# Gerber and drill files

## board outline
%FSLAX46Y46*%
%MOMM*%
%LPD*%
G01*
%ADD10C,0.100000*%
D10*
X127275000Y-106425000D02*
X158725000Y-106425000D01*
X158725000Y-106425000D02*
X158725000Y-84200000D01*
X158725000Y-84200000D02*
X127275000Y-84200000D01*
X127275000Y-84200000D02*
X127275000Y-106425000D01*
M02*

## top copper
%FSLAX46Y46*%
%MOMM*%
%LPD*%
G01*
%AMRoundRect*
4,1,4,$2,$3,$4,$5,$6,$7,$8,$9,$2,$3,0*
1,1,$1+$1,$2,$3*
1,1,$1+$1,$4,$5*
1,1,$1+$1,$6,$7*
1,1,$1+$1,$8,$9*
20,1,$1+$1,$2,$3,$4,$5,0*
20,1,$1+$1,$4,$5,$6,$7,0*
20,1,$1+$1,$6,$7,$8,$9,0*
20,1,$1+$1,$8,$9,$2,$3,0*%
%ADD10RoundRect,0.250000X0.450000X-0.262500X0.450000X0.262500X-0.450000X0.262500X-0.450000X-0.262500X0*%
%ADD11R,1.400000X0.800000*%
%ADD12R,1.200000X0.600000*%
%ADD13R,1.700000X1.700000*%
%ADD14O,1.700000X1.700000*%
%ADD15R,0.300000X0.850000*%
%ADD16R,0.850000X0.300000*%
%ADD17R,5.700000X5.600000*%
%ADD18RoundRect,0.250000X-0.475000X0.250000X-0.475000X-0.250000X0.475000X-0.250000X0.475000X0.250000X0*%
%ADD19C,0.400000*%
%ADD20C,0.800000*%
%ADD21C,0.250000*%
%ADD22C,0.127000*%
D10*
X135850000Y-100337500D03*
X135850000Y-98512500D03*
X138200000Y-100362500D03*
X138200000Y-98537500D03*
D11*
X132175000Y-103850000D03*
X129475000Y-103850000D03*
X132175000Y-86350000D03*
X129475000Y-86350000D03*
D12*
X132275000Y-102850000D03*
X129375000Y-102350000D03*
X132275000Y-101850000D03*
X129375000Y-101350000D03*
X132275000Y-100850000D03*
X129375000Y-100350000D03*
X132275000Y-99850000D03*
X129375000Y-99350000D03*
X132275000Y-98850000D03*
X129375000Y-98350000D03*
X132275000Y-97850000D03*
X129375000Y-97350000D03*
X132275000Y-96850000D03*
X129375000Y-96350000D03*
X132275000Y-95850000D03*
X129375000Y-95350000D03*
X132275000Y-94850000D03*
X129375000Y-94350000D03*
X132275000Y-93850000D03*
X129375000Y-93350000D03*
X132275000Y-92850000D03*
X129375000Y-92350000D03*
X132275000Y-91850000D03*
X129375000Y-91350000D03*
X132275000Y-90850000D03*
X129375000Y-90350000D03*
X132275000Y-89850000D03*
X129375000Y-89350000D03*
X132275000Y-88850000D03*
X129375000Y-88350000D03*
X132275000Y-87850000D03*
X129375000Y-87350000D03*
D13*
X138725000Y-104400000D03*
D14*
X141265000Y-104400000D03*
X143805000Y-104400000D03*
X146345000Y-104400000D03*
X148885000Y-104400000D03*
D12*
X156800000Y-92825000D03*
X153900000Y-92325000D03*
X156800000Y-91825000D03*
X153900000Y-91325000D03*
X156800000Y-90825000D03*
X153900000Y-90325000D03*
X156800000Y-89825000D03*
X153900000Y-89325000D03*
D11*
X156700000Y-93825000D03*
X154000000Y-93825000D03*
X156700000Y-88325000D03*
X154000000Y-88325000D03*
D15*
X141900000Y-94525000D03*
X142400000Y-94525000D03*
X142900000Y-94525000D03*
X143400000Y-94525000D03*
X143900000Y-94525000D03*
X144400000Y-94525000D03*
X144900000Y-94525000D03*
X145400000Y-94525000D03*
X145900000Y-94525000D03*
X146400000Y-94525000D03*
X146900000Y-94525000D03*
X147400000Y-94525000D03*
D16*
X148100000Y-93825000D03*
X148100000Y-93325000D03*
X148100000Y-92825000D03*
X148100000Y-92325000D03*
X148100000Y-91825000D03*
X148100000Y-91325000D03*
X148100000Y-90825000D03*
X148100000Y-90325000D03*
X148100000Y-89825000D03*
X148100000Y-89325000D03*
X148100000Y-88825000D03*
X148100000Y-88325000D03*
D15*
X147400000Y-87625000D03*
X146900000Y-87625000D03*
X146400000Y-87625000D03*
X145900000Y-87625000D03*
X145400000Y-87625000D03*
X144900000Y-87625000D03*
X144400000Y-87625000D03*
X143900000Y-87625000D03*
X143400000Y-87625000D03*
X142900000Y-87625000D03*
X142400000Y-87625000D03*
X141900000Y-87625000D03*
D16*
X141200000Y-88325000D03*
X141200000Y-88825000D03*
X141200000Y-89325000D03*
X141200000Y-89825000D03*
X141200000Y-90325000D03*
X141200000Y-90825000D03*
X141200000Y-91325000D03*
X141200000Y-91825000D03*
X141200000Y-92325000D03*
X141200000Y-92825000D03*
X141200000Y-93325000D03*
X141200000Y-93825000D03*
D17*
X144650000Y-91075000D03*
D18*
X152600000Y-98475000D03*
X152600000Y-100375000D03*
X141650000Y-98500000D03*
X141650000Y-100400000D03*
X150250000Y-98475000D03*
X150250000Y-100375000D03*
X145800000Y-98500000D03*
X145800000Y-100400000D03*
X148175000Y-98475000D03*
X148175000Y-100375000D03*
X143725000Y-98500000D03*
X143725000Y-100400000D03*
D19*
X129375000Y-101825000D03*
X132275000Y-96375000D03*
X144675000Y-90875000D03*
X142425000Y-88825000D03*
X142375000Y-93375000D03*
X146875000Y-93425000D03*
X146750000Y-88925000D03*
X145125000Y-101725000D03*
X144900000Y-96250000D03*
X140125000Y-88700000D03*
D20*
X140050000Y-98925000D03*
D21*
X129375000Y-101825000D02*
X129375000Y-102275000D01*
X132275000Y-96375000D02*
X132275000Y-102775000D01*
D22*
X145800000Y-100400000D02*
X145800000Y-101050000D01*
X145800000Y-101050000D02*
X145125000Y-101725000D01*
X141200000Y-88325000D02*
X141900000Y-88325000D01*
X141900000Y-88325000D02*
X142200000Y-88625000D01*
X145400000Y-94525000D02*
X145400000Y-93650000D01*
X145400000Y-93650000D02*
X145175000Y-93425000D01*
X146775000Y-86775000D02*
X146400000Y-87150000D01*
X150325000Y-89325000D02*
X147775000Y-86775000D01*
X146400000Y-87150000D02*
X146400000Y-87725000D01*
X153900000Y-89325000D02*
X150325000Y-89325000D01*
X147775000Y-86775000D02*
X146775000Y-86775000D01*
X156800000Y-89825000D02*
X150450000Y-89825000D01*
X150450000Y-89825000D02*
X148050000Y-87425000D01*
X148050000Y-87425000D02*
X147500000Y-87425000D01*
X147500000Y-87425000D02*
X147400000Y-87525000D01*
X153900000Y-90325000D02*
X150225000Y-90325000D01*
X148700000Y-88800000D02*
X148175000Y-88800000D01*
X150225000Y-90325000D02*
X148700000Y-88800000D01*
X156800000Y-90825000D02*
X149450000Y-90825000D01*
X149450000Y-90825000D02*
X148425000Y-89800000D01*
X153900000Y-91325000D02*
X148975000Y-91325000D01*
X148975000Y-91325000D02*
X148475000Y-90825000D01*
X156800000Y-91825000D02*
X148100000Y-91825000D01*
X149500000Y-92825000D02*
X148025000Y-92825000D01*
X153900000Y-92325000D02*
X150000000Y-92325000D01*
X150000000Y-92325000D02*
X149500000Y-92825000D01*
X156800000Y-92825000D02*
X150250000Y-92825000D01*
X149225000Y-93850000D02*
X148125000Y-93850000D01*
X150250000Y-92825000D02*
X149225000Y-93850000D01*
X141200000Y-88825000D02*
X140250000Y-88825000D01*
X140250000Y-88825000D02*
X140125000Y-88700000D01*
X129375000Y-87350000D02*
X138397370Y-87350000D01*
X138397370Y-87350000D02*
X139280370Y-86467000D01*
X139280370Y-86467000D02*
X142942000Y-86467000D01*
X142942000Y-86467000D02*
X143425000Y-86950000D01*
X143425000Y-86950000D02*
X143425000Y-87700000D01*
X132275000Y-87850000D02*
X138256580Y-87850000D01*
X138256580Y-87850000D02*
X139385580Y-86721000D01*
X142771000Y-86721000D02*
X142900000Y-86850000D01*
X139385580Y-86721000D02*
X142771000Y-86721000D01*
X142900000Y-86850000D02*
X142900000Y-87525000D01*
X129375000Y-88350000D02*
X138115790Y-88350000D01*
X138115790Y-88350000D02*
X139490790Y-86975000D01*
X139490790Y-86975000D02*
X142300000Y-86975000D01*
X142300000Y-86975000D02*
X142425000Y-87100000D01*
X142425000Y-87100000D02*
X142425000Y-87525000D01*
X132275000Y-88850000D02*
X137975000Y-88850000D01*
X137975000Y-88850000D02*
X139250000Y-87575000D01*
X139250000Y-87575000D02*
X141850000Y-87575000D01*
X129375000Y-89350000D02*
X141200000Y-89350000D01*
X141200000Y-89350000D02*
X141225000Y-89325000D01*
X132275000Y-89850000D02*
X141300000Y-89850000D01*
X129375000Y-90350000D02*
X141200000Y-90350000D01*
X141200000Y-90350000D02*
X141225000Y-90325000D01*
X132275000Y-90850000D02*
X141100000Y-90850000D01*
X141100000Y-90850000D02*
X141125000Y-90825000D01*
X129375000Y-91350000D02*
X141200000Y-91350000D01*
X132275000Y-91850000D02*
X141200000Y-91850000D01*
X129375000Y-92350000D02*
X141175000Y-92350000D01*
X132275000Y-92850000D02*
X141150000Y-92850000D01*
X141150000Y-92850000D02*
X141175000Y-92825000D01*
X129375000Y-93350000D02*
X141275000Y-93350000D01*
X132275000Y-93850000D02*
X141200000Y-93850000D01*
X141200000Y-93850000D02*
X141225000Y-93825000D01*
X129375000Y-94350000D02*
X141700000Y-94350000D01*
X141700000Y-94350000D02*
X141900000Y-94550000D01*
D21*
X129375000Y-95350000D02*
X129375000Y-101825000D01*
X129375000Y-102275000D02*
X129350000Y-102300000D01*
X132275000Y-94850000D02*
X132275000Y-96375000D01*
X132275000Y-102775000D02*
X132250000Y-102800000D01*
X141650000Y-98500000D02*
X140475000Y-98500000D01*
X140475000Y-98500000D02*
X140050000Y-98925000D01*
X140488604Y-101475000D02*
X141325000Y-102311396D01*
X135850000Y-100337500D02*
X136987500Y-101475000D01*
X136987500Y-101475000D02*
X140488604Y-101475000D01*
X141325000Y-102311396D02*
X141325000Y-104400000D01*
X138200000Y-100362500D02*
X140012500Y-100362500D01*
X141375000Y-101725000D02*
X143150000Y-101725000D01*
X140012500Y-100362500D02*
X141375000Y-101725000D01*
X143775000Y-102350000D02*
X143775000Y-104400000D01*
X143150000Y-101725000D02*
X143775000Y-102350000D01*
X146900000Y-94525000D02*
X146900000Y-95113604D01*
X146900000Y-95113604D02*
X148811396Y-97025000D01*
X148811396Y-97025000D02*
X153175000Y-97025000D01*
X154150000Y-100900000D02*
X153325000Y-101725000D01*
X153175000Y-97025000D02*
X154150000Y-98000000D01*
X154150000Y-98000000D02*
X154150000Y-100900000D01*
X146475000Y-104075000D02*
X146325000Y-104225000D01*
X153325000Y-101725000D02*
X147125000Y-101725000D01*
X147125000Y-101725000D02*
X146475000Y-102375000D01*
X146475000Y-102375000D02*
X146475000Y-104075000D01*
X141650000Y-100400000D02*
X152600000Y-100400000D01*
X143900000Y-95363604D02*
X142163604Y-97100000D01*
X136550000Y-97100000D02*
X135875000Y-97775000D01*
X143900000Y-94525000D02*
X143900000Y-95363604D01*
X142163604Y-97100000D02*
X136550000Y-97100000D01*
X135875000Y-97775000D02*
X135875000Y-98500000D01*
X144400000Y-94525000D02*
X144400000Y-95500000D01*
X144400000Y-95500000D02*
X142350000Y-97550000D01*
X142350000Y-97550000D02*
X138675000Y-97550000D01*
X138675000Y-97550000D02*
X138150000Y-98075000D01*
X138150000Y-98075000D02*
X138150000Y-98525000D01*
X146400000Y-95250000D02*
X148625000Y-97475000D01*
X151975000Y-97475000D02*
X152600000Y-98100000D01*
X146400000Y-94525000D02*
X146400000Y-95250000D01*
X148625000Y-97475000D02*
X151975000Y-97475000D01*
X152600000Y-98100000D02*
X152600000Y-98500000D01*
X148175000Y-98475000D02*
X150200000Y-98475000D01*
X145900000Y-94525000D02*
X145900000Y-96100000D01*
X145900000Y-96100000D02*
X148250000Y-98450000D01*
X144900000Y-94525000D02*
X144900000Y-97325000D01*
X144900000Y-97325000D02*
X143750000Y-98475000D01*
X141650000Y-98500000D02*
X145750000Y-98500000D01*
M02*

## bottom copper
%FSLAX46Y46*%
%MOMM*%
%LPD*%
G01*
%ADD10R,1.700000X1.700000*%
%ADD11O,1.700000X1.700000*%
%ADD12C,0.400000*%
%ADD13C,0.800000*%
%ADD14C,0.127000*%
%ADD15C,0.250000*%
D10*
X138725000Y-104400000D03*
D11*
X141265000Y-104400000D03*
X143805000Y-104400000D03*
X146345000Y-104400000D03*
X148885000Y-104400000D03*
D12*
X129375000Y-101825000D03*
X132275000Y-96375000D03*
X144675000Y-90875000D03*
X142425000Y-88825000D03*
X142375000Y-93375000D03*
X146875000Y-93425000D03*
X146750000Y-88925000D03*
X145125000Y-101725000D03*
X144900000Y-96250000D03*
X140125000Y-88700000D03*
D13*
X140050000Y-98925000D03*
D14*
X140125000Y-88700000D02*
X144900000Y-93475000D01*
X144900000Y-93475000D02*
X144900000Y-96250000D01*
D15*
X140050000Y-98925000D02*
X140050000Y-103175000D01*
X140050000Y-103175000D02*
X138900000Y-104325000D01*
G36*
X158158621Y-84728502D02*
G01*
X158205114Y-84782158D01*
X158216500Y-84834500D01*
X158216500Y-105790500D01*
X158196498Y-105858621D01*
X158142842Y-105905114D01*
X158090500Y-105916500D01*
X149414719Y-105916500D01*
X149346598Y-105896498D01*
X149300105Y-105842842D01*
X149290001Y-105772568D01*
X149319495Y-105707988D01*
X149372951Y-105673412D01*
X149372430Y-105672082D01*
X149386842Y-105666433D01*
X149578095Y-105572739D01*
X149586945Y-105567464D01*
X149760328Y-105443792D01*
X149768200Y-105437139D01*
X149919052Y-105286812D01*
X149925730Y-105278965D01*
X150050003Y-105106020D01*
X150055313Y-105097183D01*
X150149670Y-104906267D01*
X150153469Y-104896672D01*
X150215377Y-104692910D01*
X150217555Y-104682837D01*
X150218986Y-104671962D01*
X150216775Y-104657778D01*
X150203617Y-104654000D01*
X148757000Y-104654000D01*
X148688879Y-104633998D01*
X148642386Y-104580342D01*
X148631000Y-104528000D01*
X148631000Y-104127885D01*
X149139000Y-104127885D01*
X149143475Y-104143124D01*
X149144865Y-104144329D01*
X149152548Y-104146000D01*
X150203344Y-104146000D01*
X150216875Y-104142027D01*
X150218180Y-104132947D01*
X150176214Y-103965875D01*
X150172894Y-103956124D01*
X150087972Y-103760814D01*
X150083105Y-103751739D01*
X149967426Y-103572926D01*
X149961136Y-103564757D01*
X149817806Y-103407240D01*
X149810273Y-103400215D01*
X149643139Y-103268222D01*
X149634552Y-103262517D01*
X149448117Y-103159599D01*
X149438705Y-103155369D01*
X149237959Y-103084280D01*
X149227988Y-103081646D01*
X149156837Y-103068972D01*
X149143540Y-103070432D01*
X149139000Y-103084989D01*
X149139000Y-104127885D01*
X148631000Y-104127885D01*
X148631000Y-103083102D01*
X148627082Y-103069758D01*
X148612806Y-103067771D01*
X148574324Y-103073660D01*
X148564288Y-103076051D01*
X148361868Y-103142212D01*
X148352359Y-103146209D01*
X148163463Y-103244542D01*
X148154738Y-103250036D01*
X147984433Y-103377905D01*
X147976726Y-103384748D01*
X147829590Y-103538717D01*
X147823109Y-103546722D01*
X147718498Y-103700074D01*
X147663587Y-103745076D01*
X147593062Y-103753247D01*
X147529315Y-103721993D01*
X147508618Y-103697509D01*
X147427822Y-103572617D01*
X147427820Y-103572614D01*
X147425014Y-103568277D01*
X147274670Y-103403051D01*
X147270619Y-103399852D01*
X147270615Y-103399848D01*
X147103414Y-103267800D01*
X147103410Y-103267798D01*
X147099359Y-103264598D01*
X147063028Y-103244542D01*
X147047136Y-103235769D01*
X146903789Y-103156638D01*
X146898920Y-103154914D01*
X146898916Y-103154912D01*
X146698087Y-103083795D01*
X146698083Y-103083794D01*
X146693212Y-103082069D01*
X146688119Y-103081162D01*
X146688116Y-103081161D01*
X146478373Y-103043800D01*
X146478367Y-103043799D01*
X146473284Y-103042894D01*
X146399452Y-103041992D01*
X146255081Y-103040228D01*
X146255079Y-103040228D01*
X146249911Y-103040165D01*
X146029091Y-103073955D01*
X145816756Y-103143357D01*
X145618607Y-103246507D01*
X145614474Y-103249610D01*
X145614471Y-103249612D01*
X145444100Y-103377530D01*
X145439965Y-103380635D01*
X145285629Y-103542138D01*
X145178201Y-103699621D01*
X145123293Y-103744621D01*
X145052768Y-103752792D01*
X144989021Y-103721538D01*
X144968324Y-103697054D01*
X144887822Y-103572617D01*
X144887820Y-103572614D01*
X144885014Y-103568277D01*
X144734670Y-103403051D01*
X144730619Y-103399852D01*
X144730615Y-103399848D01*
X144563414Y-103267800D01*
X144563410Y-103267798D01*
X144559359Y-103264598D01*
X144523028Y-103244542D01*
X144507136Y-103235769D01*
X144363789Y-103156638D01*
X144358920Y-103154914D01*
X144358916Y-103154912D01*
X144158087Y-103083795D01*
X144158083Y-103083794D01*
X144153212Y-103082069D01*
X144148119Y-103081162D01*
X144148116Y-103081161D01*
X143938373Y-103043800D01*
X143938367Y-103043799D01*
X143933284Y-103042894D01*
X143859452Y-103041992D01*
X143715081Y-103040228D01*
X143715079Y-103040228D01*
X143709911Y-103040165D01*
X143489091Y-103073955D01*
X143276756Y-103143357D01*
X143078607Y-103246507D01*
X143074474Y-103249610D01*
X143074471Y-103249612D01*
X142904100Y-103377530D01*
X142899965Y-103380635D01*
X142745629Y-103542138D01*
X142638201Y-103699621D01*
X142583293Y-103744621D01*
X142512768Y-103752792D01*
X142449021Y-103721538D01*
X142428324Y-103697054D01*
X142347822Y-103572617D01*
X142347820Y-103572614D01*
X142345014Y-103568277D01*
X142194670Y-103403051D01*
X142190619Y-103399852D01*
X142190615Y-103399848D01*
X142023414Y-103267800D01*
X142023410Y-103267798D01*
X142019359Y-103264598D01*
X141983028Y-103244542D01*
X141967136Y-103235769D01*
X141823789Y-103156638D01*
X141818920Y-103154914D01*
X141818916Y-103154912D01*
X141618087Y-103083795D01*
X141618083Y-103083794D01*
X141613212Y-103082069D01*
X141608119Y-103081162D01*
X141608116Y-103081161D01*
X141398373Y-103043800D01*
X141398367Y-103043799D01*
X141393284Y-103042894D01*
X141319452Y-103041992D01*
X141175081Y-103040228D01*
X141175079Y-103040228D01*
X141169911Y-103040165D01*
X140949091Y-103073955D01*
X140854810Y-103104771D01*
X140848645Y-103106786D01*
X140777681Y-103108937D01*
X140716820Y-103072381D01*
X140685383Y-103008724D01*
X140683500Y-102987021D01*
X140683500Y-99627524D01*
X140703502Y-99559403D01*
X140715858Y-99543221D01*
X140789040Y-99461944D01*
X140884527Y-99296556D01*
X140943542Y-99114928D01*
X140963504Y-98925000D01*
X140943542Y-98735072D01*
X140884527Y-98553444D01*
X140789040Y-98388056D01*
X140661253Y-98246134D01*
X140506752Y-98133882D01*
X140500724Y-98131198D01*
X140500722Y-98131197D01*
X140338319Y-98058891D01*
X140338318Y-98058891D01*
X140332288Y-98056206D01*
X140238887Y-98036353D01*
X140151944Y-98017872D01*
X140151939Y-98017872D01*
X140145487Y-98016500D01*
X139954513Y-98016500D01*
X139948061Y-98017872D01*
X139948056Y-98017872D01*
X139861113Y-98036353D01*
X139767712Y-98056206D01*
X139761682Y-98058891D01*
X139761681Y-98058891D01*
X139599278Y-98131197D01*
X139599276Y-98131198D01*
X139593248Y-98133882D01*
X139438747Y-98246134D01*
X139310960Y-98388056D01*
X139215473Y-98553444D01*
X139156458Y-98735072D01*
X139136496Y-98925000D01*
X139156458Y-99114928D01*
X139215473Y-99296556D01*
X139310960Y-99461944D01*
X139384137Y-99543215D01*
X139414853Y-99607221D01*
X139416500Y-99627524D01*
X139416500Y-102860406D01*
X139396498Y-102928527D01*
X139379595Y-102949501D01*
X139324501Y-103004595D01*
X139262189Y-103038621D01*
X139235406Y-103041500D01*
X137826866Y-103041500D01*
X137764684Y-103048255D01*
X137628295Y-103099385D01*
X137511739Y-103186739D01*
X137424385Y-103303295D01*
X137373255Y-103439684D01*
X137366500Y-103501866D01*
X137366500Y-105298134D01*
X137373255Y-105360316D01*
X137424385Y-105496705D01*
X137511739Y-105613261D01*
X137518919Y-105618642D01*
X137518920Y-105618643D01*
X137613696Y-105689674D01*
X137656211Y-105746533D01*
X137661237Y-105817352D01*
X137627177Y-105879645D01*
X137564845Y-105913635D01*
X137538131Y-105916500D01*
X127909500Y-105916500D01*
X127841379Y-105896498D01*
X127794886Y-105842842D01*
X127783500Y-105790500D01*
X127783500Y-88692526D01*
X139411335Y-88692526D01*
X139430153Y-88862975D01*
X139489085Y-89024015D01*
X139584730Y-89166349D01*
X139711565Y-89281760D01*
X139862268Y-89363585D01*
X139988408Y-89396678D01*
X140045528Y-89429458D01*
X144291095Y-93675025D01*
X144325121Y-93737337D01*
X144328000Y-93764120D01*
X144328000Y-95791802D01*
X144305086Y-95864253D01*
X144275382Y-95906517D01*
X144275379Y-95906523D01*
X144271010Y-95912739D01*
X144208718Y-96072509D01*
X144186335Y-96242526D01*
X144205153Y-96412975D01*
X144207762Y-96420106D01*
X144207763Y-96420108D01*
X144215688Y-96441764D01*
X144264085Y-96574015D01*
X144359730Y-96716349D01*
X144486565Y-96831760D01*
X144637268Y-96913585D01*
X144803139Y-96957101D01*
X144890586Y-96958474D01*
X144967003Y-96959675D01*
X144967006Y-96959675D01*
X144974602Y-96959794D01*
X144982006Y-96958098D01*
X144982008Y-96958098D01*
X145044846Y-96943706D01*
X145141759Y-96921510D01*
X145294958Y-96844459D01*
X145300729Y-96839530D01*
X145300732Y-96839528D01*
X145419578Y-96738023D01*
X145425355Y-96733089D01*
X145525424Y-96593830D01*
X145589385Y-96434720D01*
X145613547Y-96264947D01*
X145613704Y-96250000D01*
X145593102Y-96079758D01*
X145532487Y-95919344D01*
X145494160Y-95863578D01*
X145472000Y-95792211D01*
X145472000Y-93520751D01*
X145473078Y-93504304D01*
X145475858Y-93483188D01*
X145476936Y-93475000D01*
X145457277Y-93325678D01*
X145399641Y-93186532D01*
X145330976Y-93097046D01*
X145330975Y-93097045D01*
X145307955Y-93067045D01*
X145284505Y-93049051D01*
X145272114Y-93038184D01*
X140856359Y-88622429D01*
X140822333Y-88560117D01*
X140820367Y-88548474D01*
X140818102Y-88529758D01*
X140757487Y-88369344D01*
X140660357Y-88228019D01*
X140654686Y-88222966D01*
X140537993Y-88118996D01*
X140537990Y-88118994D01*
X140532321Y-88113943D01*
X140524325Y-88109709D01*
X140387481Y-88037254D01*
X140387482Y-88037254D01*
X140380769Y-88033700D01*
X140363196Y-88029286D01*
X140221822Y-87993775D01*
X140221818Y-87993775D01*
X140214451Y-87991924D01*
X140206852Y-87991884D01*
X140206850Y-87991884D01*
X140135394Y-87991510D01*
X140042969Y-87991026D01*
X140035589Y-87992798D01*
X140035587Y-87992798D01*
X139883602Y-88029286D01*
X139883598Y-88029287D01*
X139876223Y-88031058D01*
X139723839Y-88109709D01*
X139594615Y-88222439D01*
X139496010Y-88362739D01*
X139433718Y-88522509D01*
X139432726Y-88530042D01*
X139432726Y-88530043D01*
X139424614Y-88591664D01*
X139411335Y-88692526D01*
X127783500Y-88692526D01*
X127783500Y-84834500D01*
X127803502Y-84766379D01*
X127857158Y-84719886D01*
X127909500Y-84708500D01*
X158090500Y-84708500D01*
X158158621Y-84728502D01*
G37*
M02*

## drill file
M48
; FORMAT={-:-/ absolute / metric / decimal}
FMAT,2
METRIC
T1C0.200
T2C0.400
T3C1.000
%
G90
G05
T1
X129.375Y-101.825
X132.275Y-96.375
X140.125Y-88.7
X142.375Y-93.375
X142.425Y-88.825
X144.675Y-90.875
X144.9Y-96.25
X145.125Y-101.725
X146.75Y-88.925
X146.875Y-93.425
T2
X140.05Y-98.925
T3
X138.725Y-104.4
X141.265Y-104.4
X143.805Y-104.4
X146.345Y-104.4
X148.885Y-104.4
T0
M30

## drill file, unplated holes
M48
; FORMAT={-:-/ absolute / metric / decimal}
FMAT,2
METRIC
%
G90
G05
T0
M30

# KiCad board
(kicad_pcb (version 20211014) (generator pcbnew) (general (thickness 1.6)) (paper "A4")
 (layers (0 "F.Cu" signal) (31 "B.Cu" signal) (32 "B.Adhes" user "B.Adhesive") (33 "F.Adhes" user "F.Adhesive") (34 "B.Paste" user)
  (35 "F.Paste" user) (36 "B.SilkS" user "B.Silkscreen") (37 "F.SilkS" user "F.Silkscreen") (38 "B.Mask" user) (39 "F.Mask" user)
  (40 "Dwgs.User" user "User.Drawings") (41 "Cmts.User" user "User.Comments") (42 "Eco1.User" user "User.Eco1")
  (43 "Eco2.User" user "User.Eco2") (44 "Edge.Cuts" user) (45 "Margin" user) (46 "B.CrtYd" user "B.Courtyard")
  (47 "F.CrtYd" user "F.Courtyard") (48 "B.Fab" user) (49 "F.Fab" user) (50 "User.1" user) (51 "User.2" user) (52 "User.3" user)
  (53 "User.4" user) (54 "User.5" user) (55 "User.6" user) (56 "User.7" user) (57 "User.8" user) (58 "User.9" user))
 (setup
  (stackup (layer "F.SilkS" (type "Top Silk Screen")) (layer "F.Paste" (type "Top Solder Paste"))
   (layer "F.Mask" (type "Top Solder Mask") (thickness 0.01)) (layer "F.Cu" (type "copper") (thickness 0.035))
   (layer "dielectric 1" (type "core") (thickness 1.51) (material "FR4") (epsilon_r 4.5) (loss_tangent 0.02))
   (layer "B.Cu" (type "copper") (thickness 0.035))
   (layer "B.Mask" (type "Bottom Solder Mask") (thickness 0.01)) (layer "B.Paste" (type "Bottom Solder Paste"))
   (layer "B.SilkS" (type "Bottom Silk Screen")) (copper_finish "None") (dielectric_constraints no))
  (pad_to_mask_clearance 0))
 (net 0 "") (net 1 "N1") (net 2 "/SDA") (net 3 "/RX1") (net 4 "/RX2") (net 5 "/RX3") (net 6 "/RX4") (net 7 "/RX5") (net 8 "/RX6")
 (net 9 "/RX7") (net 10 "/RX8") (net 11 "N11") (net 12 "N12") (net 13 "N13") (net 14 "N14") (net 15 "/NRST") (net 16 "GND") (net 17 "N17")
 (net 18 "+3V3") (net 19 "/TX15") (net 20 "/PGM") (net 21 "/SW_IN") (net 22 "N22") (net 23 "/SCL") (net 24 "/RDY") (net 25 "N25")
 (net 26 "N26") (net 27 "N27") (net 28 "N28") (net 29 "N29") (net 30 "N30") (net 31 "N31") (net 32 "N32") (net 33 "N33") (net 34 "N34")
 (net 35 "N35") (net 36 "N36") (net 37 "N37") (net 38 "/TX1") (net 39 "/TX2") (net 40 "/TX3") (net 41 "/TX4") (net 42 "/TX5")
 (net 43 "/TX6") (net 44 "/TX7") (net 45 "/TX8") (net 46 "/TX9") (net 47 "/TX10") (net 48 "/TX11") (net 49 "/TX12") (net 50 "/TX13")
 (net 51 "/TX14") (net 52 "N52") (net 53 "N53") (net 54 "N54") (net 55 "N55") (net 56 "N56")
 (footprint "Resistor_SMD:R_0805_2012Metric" (layer "F.Cu") (at 135.85 99.425 90)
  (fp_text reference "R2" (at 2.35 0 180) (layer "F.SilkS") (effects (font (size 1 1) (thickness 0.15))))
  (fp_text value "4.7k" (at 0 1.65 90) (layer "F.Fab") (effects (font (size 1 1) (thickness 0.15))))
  (pad "1" smd roundrect (at -0.9125 0 90) (size 1.025 1.4) (layers "F.Cu" "F.Paste" "F.Mask") (roundrect_rratio 0.243902) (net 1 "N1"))
  (pad "2" smd roundrect (at 0.9125 0 90) (size 1.025 1.4) (layers "F.Cu" "F.Paste" "F.Mask") (roundrect_rratio 0.243902) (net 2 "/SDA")))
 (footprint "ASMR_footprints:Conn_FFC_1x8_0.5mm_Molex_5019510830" (layer "F.Cu") (at 155.35 91.075 90)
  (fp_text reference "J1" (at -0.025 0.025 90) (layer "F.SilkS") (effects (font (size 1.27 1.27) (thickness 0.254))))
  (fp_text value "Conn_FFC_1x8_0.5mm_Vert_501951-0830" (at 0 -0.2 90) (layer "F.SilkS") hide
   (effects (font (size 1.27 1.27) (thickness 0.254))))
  (pad "1" smd rect (at -1.75 1.45 90) (size 0.6 1.2) (layers "F.Cu" "F.Paste" "F.Mask") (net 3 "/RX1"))
  (pad "2" smd rect (at -1.25 -1.45 90) (size 0.6 1.2) (layers "F.Cu" "F.Paste" "F.Mask") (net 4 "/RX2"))
  (pad "3" smd rect (at -0.75 1.45 90) (size 0.6 1.2) (layers "F.Cu" "F.Paste" "F.Mask") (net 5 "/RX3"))
  (pad "4" smd rect (at -0.25 -1.45 90) (size 0.6 1.2) (layers "F.Cu" "F.Paste" "F.Mask") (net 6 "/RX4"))
  (pad "5" smd rect (at 0.25 1.45 90) (size 0.6 1.2) (layers "F.Cu" "F.Paste" "F.Mask") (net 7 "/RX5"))
  (pad "6" smd rect (at 0.75 -1.45 90) (size 0.6 1.2) (layers "F.Cu" "F.Paste" "F.Mask") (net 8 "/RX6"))
  (pad "7" smd rect (at 1.25 1.45 90) (size 0.6 1.2) (layers "F.Cu" "F.Paste" "F.Mask") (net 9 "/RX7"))
  (pad "8" smd rect (at 1.75 -1.45 90) (size 0.6 1.2) (layers "F.Cu" "F.Paste" "F.Mask") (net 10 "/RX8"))
  (pad "MP1" smd rect (at -2.75 1.35 90) (size 0.8 1.4) (layers "F.Cu" "F.Paste" "F.Mask") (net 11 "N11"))
  (pad "MP2" smd rect (at -2.75 -1.35 90) (size 0.8 1.4) (layers "F.Cu" "F.Paste" "F.Mask") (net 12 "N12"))
  (pad "MP3" smd rect (at 2.75 1.35 90) (size 0.8 1.4) (layers "F.Cu" "F.Paste" "F.Mask") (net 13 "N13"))
  (pad "MP4" smd rect (at 2.75 -1.35 90) (size 0.8 1.4) (layers "F.Cu" "F.Paste" "F.Mask") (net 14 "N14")))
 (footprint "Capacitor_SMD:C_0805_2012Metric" (layer "F.Cu") (at 152.6 99.425 -90)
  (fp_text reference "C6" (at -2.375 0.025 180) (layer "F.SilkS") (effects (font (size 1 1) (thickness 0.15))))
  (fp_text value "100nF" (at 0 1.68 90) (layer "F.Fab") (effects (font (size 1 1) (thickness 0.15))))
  (pad "1" smd roundrect (at -0.95 0 270) (size 1 1.45) (layers "F.Cu" "F.Paste" "F.Mask") (roundrect_rratio 0.25) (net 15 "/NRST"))
  (pad "2" smd roundrect (at 0.95 0 270) (size 1 1.45) (layers "F.Cu" "F.Paste" "F.Mask") (roundrect_rratio 0.25) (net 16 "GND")))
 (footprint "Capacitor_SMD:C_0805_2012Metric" (layer "F.Cu") (at 150.25 99.425 -90)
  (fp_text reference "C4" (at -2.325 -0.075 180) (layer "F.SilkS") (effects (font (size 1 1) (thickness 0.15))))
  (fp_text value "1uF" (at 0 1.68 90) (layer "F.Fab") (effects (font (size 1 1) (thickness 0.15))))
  (pad "1" smd roundrect (at -0.95 0 270) (size 1 1.45) (layers "F.Cu" "F.Paste" "F.Mask") (roundrect_rratio 0.25) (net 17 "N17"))
  (pad "2" smd roundrect (at 0.95 0 270) (size 1 1.45) (layers "F.Cu" "F.Paste" "F.Mask") (roundrect_rratio 0.25) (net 16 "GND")))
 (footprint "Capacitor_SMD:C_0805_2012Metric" (layer "F.Cu") (at 143.725 99.45 -90)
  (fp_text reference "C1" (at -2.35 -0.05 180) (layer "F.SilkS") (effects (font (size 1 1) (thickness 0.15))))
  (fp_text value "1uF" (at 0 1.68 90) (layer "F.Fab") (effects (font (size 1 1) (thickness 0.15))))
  (pad "1" smd roundrect (at -0.95 0 270) (size 1 1.45) (layers "F.Cu" "F.Paste" "F.Mask") (roundrect_rratio 0.25) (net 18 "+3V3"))
  (pad "2" smd roundrect (at 0.95 0 270) (size 1 1.45) (layers "F.Cu" "F.Paste" "F.Mask") (roundrect_rratio 0.25) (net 16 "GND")))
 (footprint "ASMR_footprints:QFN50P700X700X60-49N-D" (layer "F.Cu") (at 144.65 91.075 90)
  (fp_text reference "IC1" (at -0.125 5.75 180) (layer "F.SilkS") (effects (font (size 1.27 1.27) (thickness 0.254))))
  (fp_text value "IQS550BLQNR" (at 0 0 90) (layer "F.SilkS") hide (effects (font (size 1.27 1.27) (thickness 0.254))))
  (pad "1" smd rect (at -3.45 -2.75 180) (size 0.3 0.85) (layers "F.Cu" "F.Paste" "F.Mask") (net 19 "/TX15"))
  (pad "2" smd rect (at -3.45 -2.25 180) (size 0.3 0.85) (layers "F.Cu" "F.Paste" "F.Mask") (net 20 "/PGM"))
  (pad "3" smd rect (at -3.45 -1.75 180) (size 0.3 0.85) (layers "F.Cu" "F.Paste" "F.Mask") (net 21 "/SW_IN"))
  (pad "4" smd rect (at -3.45 -1.25 180) (size 0.3 0.85) (layers "F.Cu" "F.Paste" "F.Mask") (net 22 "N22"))
  (pad "5" smd rect (at -3.45 -0.75 180) (size 0.3 0.85) (layers "F.Cu" "F.Paste" "F.Mask") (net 2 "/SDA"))
  (pad "6" smd rect (at -3.45 -0.25 180) (size 0.3 0.85) (layers "F.Cu" "F.Paste" "F.Mask") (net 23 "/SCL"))
  (pad "7" smd rect (at -3.45 0.25 180) (size 0.3 0.85) (layers "F.Cu" "F.Paste" "F.Mask") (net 18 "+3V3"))
  (pad "8" smd rect (at -3.45 0.75 180) (size 0.3 0.85) (layers "F.Cu" "F.Paste" "F.Mask") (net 16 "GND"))
  (pad "9" smd rect (at -3.45 1.25 180) (size 0.3 0.85) (layers "F.Cu" "F.Paste" "F.Mask") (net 17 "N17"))
  (pad "10" smd rect (at -3.45 1.75 180) (size 0.3 0.85) (layers "F.Cu" "F.Paste" "F.Mask") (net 15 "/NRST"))
  (pad "11" smd rect (at -3.45 2.25 180) (size 0.3 0.85) (layers "F.Cu" "F.Paste" "F.Mask") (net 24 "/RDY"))
  (pad "12" smd rect (at -3.45 2.75 180) (size 0.3 0.85) (layers "F.Cu" "F.Paste" "F.Mask") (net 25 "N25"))
  (pad "13" smd rect (at -2.75 3.45 90) (size 0.3 0.85) (layers "F.Cu" "F.Paste" "F.Mask") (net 3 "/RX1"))
  (pad "14" smd rect (at -2.25 3.45 90) (size 0.3 0.85) (layers "F.Cu" "F.Paste" "F.Mask") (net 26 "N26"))
  (pad "15" smd rect (at -1.75 3.45 90) (size 0.3 0.85) (layers "F.Cu" "F.Paste" "F.Mask") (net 4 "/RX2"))
  (pad "16" smd rect (at -1.25 3.45 90) (size 0.3 0.85) (layers "F.Cu" "F.Paste" "F.Mask") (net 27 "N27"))
  (pad "17" smd rect (at -0.75 3.45 90) (size 0.3 0.85) (layers "F.Cu" "F.Paste" "F.Mask") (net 5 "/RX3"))
  (pad "18" smd rect (at -0.25 3.45 90) (size 0.3 0.85) (layers "F.Cu" "F.Paste" "F.Mask") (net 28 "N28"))
  (pad "19" smd rect (at 0.25 3.45 90) (size 0.3 0.85) (layers "F.Cu" "F.Paste" "F.Mask") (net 6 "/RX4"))
  (pad "20" smd rect (at 0.75 3.45 90) (size 0.3 0.85) (layers "F.Cu" "F.Paste" "F.Mask") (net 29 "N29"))
  (pad "21" smd rect (at 1.25 3.45 90) (size 0.3 0.85) (layers "F.Cu" "F.Paste" "F.Mask") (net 7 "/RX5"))
  (pad "22" smd rect (at 1.75 3.45 90) (size 0.3 0.85) (layers "F.Cu" "F.Paste" "F.Mask") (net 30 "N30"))
  (pad "23" smd rect (at 2.25 3.45 90) (size 0.3 0.85) (layers "F.Cu" "F.Paste" "F.Mask") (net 8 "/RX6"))
  (pad "24" smd rect (at 2.75 3.45 90) (size 0.3 0.85) (layers "F.Cu" "F.Paste" "F.Mask") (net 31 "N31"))
  (pad "25" smd rect (at 3.45 2.75 180) (size 0.3 0.85) (layers "F.Cu" "F.Paste" "F.Mask") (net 9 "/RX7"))
  (pad "26" smd rect (at 3.45 2.25 180) (size 0.3 0.85) (layers "F.Cu" "F.Paste" "F.Mask") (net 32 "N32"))
  (pad "27" smd rect (at 3.45 1.75 180) (size 0.3 0.85) (layers "F.Cu" "F.Paste" "F.Mask") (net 10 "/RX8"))
  (pad "28" smd rect (at 3.45 1.25 180) (size 0.3 0.85) (layers "F.Cu" "F.Paste" "F.Mask") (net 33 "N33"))
  (pad "29" smd rect (at 3.45 0.75 180) (size 0.3 0.85) (layers "F.Cu" "F.Paste" "F.Mask") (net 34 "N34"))
  (pad "30" smd rect (at 3.45 0.25 180) (size 0.3 0.85) (layers "F.Cu" "F.Paste" "F.Mask") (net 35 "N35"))
  (pad "31" smd rect (at 3.45 -0.25 180) (size 0.3 0.85) (layers "F.Cu" "F.Paste" "F.Mask") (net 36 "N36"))
  (pad "32" smd rect (at 3.45 -0.75 180) (size 0.3 0.85) (layers "F.Cu" "F.Paste" "F.Mask") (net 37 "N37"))
  (pad "33" smd rect (at 3.45 -1.25 180) (size 0.3 0.85) (layers "F.Cu" "F.Paste" "F.Mask") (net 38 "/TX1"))
  (pad "34" smd rect (at 3.45 -1.75 180) (size 0.3 0.85) (layers "F.Cu" "F.Paste" "F.Mask") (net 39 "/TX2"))
  (pad "35" smd rect (at 3.45 -2.25 180) (size 0.3 0.85) (layers "F.Cu" "F.Paste" "F.Mask") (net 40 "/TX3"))
  (pad "36" smd rect (at 3.45 -2.75 180) (size 0.3 0.85) (layers "F.Cu" "F.Paste" "F.Mask") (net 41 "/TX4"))
  (pad "37" smd rect (at 2.75 -3.45 90) (size 0.3 0.85) (layers "F.Cu" "F.Paste" "F.Mask") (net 16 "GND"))
  (pad "38" smd rect (at 2.25 -3.45 90) (size 0.3 0.85) (layers "F.Cu" "F.Paste" "F.Mask") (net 18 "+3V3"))
  (pad "39" smd rect (at 1.75 -3.45 90) (size 0.3 0.85) (layers "F.Cu" "F.Paste" "F.Mask") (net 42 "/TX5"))
  (pad "40" smd rect (at 1.25 -3.45 90) (size 0.3 0.85) (layers "F.Cu" "F.Paste" "F.Mask") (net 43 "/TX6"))
  (pad "41" smd rect (at 0.75 -3.45 90) (size 0.3 0.85) (layers "F.Cu" "F.Paste" "F.Mask") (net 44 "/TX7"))
  (pad "42" smd rect (at 0.25 -3.45 90) (size 0.3 0.85) (layers "F.Cu" "F.Paste" "F.Mask") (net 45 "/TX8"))
  (pad "43" smd rect (at -0.25 -3.45 90) (size 0.3 0.85) (layers "F.Cu" "F.Paste" "F.Mask") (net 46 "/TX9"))
  (pad "44" smd rect (at -0.75 -3.45 90) (size 0.3 0.85) (layers "F.Cu" "F.Paste" "F.Mask") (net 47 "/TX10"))
  (pad "45" smd rect (at -1.25 -3.45 90) (size 0.3 0.85) (layers "F.Cu" "F.Paste" "F.Mask") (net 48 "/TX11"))
  (pad "46" smd rect (at -1.75 -3.45 90) (size 0.3 0.85) (layers "F.Cu" "F.Paste" "F.Mask") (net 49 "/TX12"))
  (pad "47" smd rect (at -2.25 -3.45 90) (size 0.3 0.85) (layers "F.Cu" "F.Paste" "F.Mask") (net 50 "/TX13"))
  (pad "48" smd rect (at -2.75 -3.45 90) (size 0.3 0.85) (layers "F.Cu" "F.Paste" "F.Mask") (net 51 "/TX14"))
  (pad "49" smd rect (at 0 0 90) (size 5.6 5.7) (layers "F.Cu" "F.Paste" "F.Mask") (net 16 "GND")))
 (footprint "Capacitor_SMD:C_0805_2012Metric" (layer "F.Cu") (at 148.175 99.425 -90)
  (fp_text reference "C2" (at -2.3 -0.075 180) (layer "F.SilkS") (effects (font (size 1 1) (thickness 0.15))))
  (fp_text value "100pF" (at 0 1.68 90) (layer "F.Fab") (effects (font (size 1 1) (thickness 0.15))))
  (pad "1" smd roundrect (at -0.95 0 270) (size 1 1.45) (layers "F.Cu" "F.Paste" "F.Mask") (roundrect_rratio 0.25) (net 17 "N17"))
  (pad "2" smd roundrect (at 0.95 0 270) (size 1 1.45) (layers "F.Cu" "F.Paste" "F.Mask") (roundrect_rratio 0.25) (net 16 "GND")))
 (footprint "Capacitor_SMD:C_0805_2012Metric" (layer "F.Cu") (at 141.65 99.45 -90)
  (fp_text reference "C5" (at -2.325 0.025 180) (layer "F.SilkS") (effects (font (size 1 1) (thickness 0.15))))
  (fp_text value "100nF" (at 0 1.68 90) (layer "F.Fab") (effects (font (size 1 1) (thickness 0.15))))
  (pad "1" smd roundrect (at -0.95 0 270) (size 1 1.45) (layers "F.Cu" "F.Paste" "F.Mask") (roundrect_rratio 0.25) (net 18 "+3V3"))
  (pad "2" smd roundrect (at 0.95 0 270) (size 1 1.45) (layers "F.Cu" "F.Paste" "F.Mask") (roundrect_rratio 0.25) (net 16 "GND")))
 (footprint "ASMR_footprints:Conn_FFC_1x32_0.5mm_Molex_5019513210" (layer "F.Cu") (at 130.825 95.1 -90)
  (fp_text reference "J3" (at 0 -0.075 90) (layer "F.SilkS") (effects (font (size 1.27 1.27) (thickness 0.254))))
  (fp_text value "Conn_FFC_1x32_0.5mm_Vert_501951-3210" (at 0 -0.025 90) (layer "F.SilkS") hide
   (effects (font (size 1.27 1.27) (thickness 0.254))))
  (pad "1" smd rect (at -7.75 1.45 270) (size 0.6 1.2) (layers "F.Cu" "F.Paste" "F.Mask") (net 38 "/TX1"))
  (pad "2" smd rect (at -7.25 -1.45 270) (size 0.6 1.2) (layers "F.Cu" "F.Paste" "F.Mask") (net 39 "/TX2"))
  (pad "3" smd rect (at -6.75 1.45 270) (size 0.6 1.2) (layers "F.Cu" "F.Paste" "F.Mask") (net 40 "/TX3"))
  (pad "4" smd rect (at -6.25 -1.45 270) (size 0.6 1.2) (layers "F.Cu" "F.Paste" "F.Mask") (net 41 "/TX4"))
  (pad "5" smd rect (at -5.75 1.45 270) (size 0.6 1.2) (layers "F.Cu" "F.Paste" "F.Mask") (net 42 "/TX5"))
  (pad "6" smd rect (at -5.25 -1.45 270) (size 0.6 1.2) (layers "F.Cu" "F.Paste" "F.Mask") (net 43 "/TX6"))
  (pad "7" smd rect (at -4.75 1.45 270) (size 0.6 1.2) (layers "F.Cu" "F.Paste" "F.Mask") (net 44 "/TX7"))
  (pad "8" smd rect (at -4.25 -1.45 270) (size 0.6 1.2) (layers "F.Cu" "F.Paste" "F.Mask") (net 45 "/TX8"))
  (pad "9" smd rect (at -3.75 1.45 270) (size 0.6 1.2) (layers "F.Cu" "F.Paste" "F.Mask") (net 46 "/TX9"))
  (pad "10" smd rect (at -3.25 -1.45 270) (size 0.6 1.2) (layers "F.Cu" "F.Paste" "F.Mask") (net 47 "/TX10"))
  (pad "11" smd rect (at -2.75 1.45 270) (size 0.6 1.2) (layers "F.Cu" "F.Paste" "F.Mask") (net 48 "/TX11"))
  (pad "12" smd rect (at -2.25 -1.45 270) (size 0.6 1.2) (layers "F.Cu" "F.Paste" "F.Mask") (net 49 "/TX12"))
  (pad "13" smd rect (at -1.75 1.45 270) (size 0.6 1.2) (layers "F.Cu" "F.Paste" "F.Mask") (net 50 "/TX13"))
  (pad "14" smd rect (at -1.25 -1.45 270) (size 0.6 1.2) (layers "F.Cu" "F.Paste" "F.Mask") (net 51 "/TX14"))
  (pad "15" smd rect (at -0.75 1.45 270) (size 0.6 1.2) (layers "F.Cu" "F.Paste" "F.Mask") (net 19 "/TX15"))
  (pad "16" smd rect (at -0.25 -1.45 270) (size 0.6 1.2) (layers "F.Cu" "F.Paste" "F.Mask") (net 16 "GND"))
  (pad "17" smd rect (at 0.25 1.45 270) (size 0.6 1.2) (layers "F.Cu" "F.Paste" "F.Mask") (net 16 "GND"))
  (pad "18" smd rect (at 0.75 -1.45 270) (size 0.6 1.2) (layers "F.Cu" "F.Paste" "F.Mask") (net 16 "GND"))
  (pad "19" smd rect (at 1.25 1.45 270) (size 0.6 1.2) (layers "F.Cu" "F.Paste" "F.Mask") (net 16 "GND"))
  (pad "20" smd rect (at 1.75 -1.45 270) (size 0.6 1.2) (layers "F.Cu" "F.Paste" "F.Mask") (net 16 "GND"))
  (pad "21" smd rect (at 2.25 1.45 270) (size 0.6 1.2) (layers "F.Cu" "F.Paste" "F.Mask") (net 16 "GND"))
  (pad "22" smd rect (at 2.75 -1.45 270) (size 0.6 1.2) (layers "F.Cu" "F.Paste" "F.Mask") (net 16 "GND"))
  (pad "23" smd rect (at 3.25 1.45 270) (size 0.6 1.2) (layers "F.Cu" "F.Paste" "F.Mask") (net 16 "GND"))
  (pad "24" smd rect (at 3.75 -1.45 270) (size 0.6 1.2) (layers "F.Cu" "F.Paste" "F.Mask") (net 16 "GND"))
  (pad "25" smd rect (at 4.25 1.45 270) (size 0.6 1.2) (layers "F.Cu" "F.Paste" "F.Mask") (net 16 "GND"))
  (pad "26" smd rect (at 4.75 -1.45 270) (size 0.6 1.2) (layers "F.Cu" "F.Paste" "F.Mask") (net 16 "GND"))
  (pad "27" smd rect (at 5.25 1.45 270) (size 0.6 1.2) (layers "F.Cu" "F.Paste" "F.Mask") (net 16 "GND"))
  (pad "28" smd rect (at 5.75 -1.45 270) (size 0.6 1.2) (layers "F.Cu" "F.Paste" "F.Mask") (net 16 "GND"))
  (pad "29" smd rect (at 6.25 1.45 270) (size 0.6 1.2) (layers "F.Cu" "F.Paste" "F.Mask") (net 16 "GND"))
  (pad "30" smd rect (at 6.75 -1.45 270) (size 0.6 1.2) (layers "F.Cu" "F.Paste" "F.Mask") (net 16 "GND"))
  (pad "31" smd rect (at 7.25 1.45 270) (size 0.6 1.2) (layers "F.Cu" "F.Paste" "F.Mask") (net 16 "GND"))
  (pad "32" smd rect (at 7.75 -1.45 270) (size 0.6 1.2) (layers "F.Cu" "F.Paste" "F.Mask") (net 16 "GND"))
  (pad "MP1" smd rect (at -8.75 1.35 270) (size 0.8 1.4) (layers "F.Cu" "F.Paste" "F.Mask") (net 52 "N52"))
  (pad "MP2" smd rect (at -8.75 -1.35 270) (size 0.8 1.4) (layers "F.Cu" "F.Paste" "F.Mask") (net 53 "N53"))
  (pad "MP3" smd rect (at 8.75 1.35 270) (size 0.8 1.4) (layers "F.Cu" "F.Paste" "F.Mask") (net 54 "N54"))
  (pad "MP4" smd rect (at 8.75 -1.35 270) (size 0.8 1.4) (layers "F.Cu" "F.Paste" "F.Mask") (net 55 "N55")))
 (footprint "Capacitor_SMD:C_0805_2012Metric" (layer "F.Cu") (at 145.8 99.45 -90)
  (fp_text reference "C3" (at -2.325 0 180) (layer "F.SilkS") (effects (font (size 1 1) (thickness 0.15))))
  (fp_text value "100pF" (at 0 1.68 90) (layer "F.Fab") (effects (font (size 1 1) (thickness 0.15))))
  (pad "1" smd roundrect (at -0.95 0 270) (size 1 1.45) (layers "F.Cu" "F.Paste" "F.Mask") (roundrect_rratio 0.25) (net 18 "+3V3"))
  (pad "2" smd roundrect (at 0.95 0 270) (size 1 1.45) (layers "F.Cu" "F.Paste" "F.Mask") (roundrect_rratio 0.25) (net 16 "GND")))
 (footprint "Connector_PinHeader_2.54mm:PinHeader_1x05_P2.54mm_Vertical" (layer "F.Cu") (at 138.725 104.4 90)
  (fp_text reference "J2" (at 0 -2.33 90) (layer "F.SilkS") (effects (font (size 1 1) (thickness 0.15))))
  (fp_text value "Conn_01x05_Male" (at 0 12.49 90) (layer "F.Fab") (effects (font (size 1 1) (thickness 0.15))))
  (pad "1" thru_hole rect (at 0 0 90) (size 1.7 1.7) (drill 1) (layers *.Cu *.Mask) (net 18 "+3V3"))
  (pad "2" thru_hole oval (at 0 2.54 90) (size 1.7 1.7) (drill 1) (layers *.Cu *.Mask) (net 1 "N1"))
  (pad "3" thru_hole oval (at 0 5.08 90) (size 1.7 1.7) (drill 1) (layers *.Cu *.Mask) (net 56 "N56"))
  (pad "4" thru_hole oval (at 0 7.62 90) (size 1.7 1.7) (drill 1) (layers *.Cu *.Mask) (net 24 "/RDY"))
  (pad "5" thru_hole oval (at 0 10.16 90) (size 1.7 1.7) (drill 1) (layers *.Cu *.Mask) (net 16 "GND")))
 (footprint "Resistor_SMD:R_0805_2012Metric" (layer "F.Cu") (at 138.2 99.45 90)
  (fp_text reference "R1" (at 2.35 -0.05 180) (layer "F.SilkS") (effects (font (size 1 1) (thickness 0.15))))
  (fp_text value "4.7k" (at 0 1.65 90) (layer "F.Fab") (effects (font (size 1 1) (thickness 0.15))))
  (pad "1" smd roundrect (at -0.9125 0 90) (size 1.025 1.4) (layers "F.Cu" "F.Paste" "F.Mask") (roundrect_rratio 0.243902) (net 56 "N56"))
  (pad "2" smd roundrect (at 0.9125 0 90) (size 1.025 1.4) (layers "F.Cu" "F.Paste" "F.Mask") (roundrect_rratio 0.243902) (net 23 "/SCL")))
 (gr_rect (start 127.275 106.425) (end 158.725 84.2) (layer "Edge.Cuts") (width 0.1) (fill none))
 (segment (start 141.2 88.825) (end 140.25 88.825) (width 0.127) (layer "F.Cu") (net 18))
 (segment (start 141.65 98.5) (end 140.475 98.5) (width 0.25) (layer "F.Cu") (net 18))
 (segment (start 144.9 97.325) (end 143.75 98.475) (width 0.25) (layer "F.Cu") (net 18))
 (segment (start 144.9 94.525) (end 144.9 97.325) (width 0.25) (layer "F.Cu") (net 18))
 (segment (start 140.25 88.825) (end 140.125 88.7) (width 0.127) (layer "F.Cu") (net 18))
 (segment (start 141.65 98.5) (end 145.75 98.5) (width 0.25) (layer "F.Cu") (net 18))
 (segment (start 140.475 98.5) (end 140.05 98.925) (width 0.25) (layer "F.Cu") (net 18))
 (via (at 140.05 98.925) (size 0.8) (drill 0.4) (layers "F.Cu" "B.Cu") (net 18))
 (via (at 140.125 88.7) (size 0.4) (drill 0.2) (layers "F.Cu" "B.Cu") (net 18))
 (via (at 144.9 96.25) (size 0.4) (drill 0.2) (layers "F.Cu" "B.Cu") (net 18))
 (segment (start 140.05 98.925) (end 140.05 103.175) (width 0.25) (layer "B.Cu") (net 18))
 (segment (start 140.125 88.7) (end 144.9 93.475) (width 0.127) (layer "B.Cu") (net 18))
 (segment (start 140.05 103.175) (end 138.9 104.325) (width 0.25) (layer "B.Cu") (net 18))
 (segment (start 144.9 93.475) (end 144.9 96.25) (width 0.127) (layer "B.Cu") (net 18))
 (segment (start 145.8 101.05) (end 145.125 101.725) (width 0.127) (layer "F.Cu") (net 16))
 (segment (start 129.375 95.35) (end 129.375 101.825) (width 0.25) (layer "F.Cu") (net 16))
 (segment (start 145.4 93.65) (end 145.175 93.425) (width 0.127) (layer "F.Cu") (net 16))
 (segment (start 141.2 88.325) (end 141.9 88.325) (width 0.127) (layer "F.Cu") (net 16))
 (segment (start 132.275 96.375) (end 132.275 102.775) (width 0.25) (layer "F.Cu") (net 16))
 (segment (start 141.9 88.325) (end 142.2 88.625) (width 0.127) (layer "F.Cu") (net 16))
 (segment (start 132.275 94.85) (end 132.275 96.375) (width 0.25) (layer "F.Cu") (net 16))
 (segment (start 145.4 94.525) (end 145.4 93.65) (width 0.127) (layer "F.Cu") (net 16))
 (segment (start 132.275 102.775) (end 132.25 102.8) (width 0.25) (layer "F.Cu") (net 16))
 (segment (start 141.65 100.4) (end 152.6 100.4) (width 0.25) (layer "F.Cu") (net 16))
 (segment (start 145.8 100.4) (end 145.8 101.05) (width 0.127) (layer "F.Cu") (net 16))
 (segment (start 129.375 102.275) (end 129.35 102.3) (width 0.25) (layer "F.Cu") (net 16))
 (segment (start 129.375 101.825) (end 129.375 102.275) (width 0.25) (layer "F.Cu") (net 16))
 (via (at 145.125 101.725) (size 0.4) (drill 0.2) (layers "F.Cu" "B.Cu") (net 16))
 (via (at 146.75 88.925) (size 0.4) (drill 0.2) (layers "F.Cu" "B.Cu") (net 16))
 (via (at 142.375 93.375) (size 0.4) (drill 0.2) (layers "F.Cu" "B.Cu") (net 16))
 (via (at 142.425 88.825) (size 0.4) (drill 0.2) (layers "F.Cu" "B.Cu") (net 16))
 (via (at 132.275 96.375) (size 0.4) (drill 0.2) (layers "F.Cu" "B.Cu") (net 16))
 (via (at 144.675 90.875) (size 0.4) (drill 0.2) (layers "F.Cu" "B.Cu") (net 16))
 (via (at 146.875 93.425) (size 0.4) (drill 0.2) (layers "F.Cu" "B.Cu") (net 16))
 (via (at 129.375 101.825) (size 0.4) (drill 0.2) (layers "F.Cu" "B.Cu") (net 16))
 (segment (start 145.9 96.1) (end 148.25 98.45) (width 0.25) (layer "F.Cu") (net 17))
 (segment (start 145.9 94.525) (end 145.9 96.1) (width 0.25) (layer "F.Cu") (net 17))
 (segment (start 148.175 98.475) (end 150.2 98.475) (width 0.25) (layer "F.Cu") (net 17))
 (segment (start 152.6 98.1) (end 152.6 98.5) (width 0.25) (layer "F.Cu") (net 15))
 (segment (start 148.625 97.475) (end 151.975 97.475) (width 0.25) (layer "F.Cu") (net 15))
 (segment (start 146.4 95.25) (end 148.625 97.475) (width 0.25) (layer "F.Cu") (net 15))
 (segment (start 146.4 94.525) (end 146.4 95.25) (width 0.25) (layer "F.Cu") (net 15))
 (segment (start 151.975 97.475) (end 152.6 98.1) (width 0.25) (layer "F.Cu") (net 15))
 (segment (start 141.7 94.35) (end 141.9 94.55) (width 0.127) (layer "F.Cu") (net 19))
 (segment (start 129.375 94.35) (end 141.7 94.35) (width 0.127) (layer "F.Cu") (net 19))
 (segment (start 135.875 97.775) (end 135.875 98.5) (width 0.25) (layer "F.Cu") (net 2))
 (segment (start 143.9 95.363604) (end 142.163604 97.1) (width 0.25) (layer "F.Cu") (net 2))
 (segment (start 142.163604 97.1) (end 136.55 97.1) (width 0.25) (layer "F.Cu") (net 2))
 (segment (start 136.55 97.1) (end 135.875 97.775) (width 0.25) (layer "F.Cu") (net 2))
 (segment (start 143.9 94.525) (end 143.9 95.363604) (width 0.25) (layer "F.Cu") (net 2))
 (segment (start 144.4 95.5) (end 142.35 97.55) (width 0.25) (layer "F.Cu") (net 23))
 (segment (start 142.35 97.55) (end 138.675 97.55) (width 0.25) (layer "F.Cu") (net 23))
 (segment (start 138.15 98.075) (end 138.15 98.525) (width 0.25) (layer "F.Cu") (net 23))
 (segment (start 144.4 94.525) (end 144.4 95.5) (width 0.25) (layer "F.Cu") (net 23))
 (segment (start 138.675 97.55) (end 138.15 98.075) (width 0.25) (layer "F.Cu") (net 23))
 (segment (start 146.475 102.375) (end 146.475 104.075) (width 0.25) (layer "F.Cu") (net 24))
 (segment (start 147.125 101.725) (end 146.475 102.375) (width 0.25) (layer "F.Cu") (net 24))
 (segment (start 153.325 101.725) (end 147.125 101.725) (width 0.25) (layer "F.Cu") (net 24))
 (segment (start 146.475 104.075) (end 146.325 104.225) (width 0.25) (layer "F.Cu") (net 24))
 (segment (start 148.811396 97.025) (end 153.175 97.025) (width 0.25) (layer "F.Cu") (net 24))
 (segment (start 154.15 100.9) (end 153.325 101.725) (width 0.25) (layer "F.Cu") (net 24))
 (segment (start 153.175 97.025) (end 154.15 98) (width 0.25) (layer "F.Cu") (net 24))
 (segment (start 146.9 95.113604) (end 148.811396 97.025) (width 0.25) (layer "F.Cu") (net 24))
 (segment (start 154.15 98) (end 154.15 100.9) (width 0.25) (layer "F.Cu") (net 24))
 (segment (start 146.9 94.525) (end 146.9 95.113604) (width 0.25) (layer "F.Cu") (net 24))
 (segment (start 150.25 92.825) (end 149.225 93.85) (width 0.127) (layer "F.Cu") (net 3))
 (segment (start 149.225 93.85) (end 148.125 93.85) (width 0.127) (layer "F.Cu") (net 3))
 (segment (start 156.8 92.825) (end 150.25 92.825) (width 0.127) (layer "F.Cu") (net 3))
 (segment (start 149.5 92.825) (end 148.025 92.825) (width 0.127) (layer "F.Cu") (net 4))
 (segment (start 153.9 92.325) (end 150 92.325) (width 0.127) (layer "F.Cu") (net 4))
 (segment (start 150 92.325) (end 149.5 92.825) (width 0.127) (layer "F.Cu") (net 4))
 (segment (start 156.8 91.825) (end 148.1 91.825) (width 0.127) (layer "F.Cu") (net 5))
 (segment (start 153.9 91.325) (end 148.975 91.325) (width 0.127) (layer "F.Cu") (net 6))
 (segment (start 148.975 91.325) (end 148.475 90.825) (width 0.127) (layer "F.Cu") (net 6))
 (segment (start 149.45 90.825) (end 148.425 89.8) (width 0.127) (layer "F.Cu") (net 7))
 (segment (start 156.8 90.825) (end 149.45 90.825) (width 0.127) (layer "F.Cu") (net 7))
 (segment (start 148.7 88.8) (end 148.175 88.8) (width 0.127) (layer "F.Cu") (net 8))
 (segment (start 153.9 90.325) (end 150.225 90.325) (width 0.127) (layer "F.Cu") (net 8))
 (segment (start 150.225 90.325) (end 148.7 88.8) (width 0.127) (layer "F.Cu") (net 8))
 (segment (start 147.5 87.425) (end 147.4 87.525) (width 0.127) (layer "F.Cu") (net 9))
 (segment (start 150.45 89.825) (end 148.05 87.425) (width 0.127) (layer "F.Cu") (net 9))
 (segment (start 156.8 89.825) (end 150.45 89.825) (width 0.127) (layer "F.Cu") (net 9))
 (segment (start 148.05 87.425) (end 147.5 87.425) (width 0.127) (layer "F.Cu") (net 9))
 (segment (start 146.775 86.775) (end 146.4 87.15) (width 0.127) (layer "F.Cu") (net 10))
 (segment (start 146.4 87.15) (end 146.4 87.725) (width 0.127) (layer "F.Cu") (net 10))
 (segment (start 150.325 89.325) (end 147.775 86.775) (width 0.127) (layer "F.Cu") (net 10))
 (segment (start 153.9 89.325) (end 150.325 89.325) (width 0.127) (layer "F.Cu") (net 10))
 (segment (start 147.775 86.775) (end 146.775 86.775) (width 0.127) (layer "F.Cu") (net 10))
 (segment (start 139.28037 86.467) (end 142.942 86.467) (width 0.127) (layer "F.Cu") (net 38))
 (segment (start 142.942 86.467) (end 143.425 86.95) (width 0.127) (layer "F.Cu") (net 38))
 (segment (start 143.425 86.95) (end 143.425 87.7) (width 0.127) (layer "F.Cu") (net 38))
 (segment (start 129.375 87.35) (end 138.39737 87.35) (width 0.127) (layer "F.Cu") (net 38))
 (segment (start 138.39737 87.35) (end 139.28037 86.467) (width 0.127) (layer "F.Cu") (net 38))
 (segment (start 142.9 86.85) (end 142.9 87.525) (width 0.127) (layer "F.Cu") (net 39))
 (segment (start 142.771 86.721) (end 142.9 86.85) (width 0.127) (layer "F.Cu") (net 39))
 (segment (start 132.275 87.85) (end 138.25658 87.85) (width 0.127) (layer "F.Cu") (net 39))
 (segment (start 138.25658 87.85) (end 139.38558 86.721) (width 0.127) (layer "F.Cu") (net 39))
 (segment (start 139.38558 86.721) (end 142.771 86.721) (width 0.127) (layer "F.Cu") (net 39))
 (segment (start 139.49079 86.975) (end 142.3 86.975) (width 0.127) (layer "F.Cu") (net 40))
 (segment (start 142.3 86.975) (end 142.425 87.1) (width 0.127) (layer "F.Cu") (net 40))
 (segment (start 142.425 87.1) (end 142.425 87.525) (width 0.127) (layer "F.Cu") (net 40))
 (segment (start 129.375 88.35) (end 138.11579 88.35) (width 0.127) (layer "F.Cu") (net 40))
 (segment (start 138.11579 88.35) (end 139.49079 86.975) (width 0.127) (layer "F.Cu") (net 40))
 (segment (start 137.975 88.85) (end 139.25 87.575) (width 0.127) (layer "F.Cu") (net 41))
 (segment (start 132.275 88.85) (end 137.975 88.85) (width 0.127) (layer "F.Cu") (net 41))
 (segment (start 139.25 87.575) (end 141.85 87.575) (width 0.127) (layer "F.Cu") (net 41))
 (segment (start 141.2 89.35) (end 141.225 89.325) (width 0.127) (layer "F.Cu") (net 42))
 (segment (start 129.375 89.35) (end 141.2 89.35) (width 0.127) (layer "F.Cu") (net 42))
 (segment (start 132.275 89.85) (end 141.3 89.85) (width 0.127) (layer "F.Cu") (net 43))
 (segment (start 129.375 90.35) (end 141.2 90.35) (width 0.127) (layer "F.Cu") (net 44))
 (segment (start 141.2 90.35) (end 141.225 90.325) (width 0.127) (layer "F.Cu") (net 44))
 (segment (start 141.1 90.85) (end 141.125 90.825) (width 0.127) (layer "F.Cu") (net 45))
 (segment (start 132.275 90.85) (end 141.1 90.85) (width 0.127) (layer "F.Cu") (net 45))
 (segment (start 129.375 91.35) (end 141.2 91.35) (width 0.127) (layer "F.Cu") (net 46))
 (segment (start 132.275 91.85) (end 141.2 91.85) (width 0.127) (layer "F.Cu") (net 47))
 (segment (start 129.375 92.35) (end 141.175 92.35) (width 0.127) (layer "F.Cu") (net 48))
 (segment (start 132.275 92.85) (end 141.15 92.85) (width 0.127) (layer "F.Cu") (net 49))
 (segment (start 141.15 92.85) (end 141.175 92.825) (width 0.127) (layer "F.Cu") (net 49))
 (segment (start 129.375 93.35) (end 141.275 93.35) (width 0.127) (layer "F.Cu") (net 50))
 (segment (start 141.2 93.85) (end 141.225 93.825) (width 0.127) (layer "F.Cu") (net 51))
 (segment (start 132.275 93.85) (end 141.2 93.85) (width 0.127) (layer "F.Cu") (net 51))
 (segment (start 136.9875 101.475) (end 140.488604 101.475) (width 0.25) (layer "F.Cu") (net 1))
 (segment (start 141.325 102.311396) (end 141.325 104.4) (width 0.25) (layer "F.Cu") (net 1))
 (segment (start 135.85 100.3375) (end 136.9875 101.475) (width 0.25) (layer "F.Cu") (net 1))
 (segment (start 140.488604 101.475) (end 141.325 102.311396) (width 0.25) (layer "F.Cu") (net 1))
 (segment (start 143.15 101.725) (end 143.775 102.35) (width 0.25) (layer "F.Cu") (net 56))
 (segment (start 143.775 102.35) (end 143.775 104.4) (width 0.25) (layer "F.Cu") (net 56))
 (segment (start 141.375 101.725) (end 143.15 101.725) (width 0.25) (layer "F.Cu") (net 56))
 (segment (start 140.0125 100.3625) (end 141.375 101.725) (width 0.25) (layer "F.Cu") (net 56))
 (segment (start 138.2 100.3625) (end 140.0125 100.3625) (width 0.25) (layer "F.Cu") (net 56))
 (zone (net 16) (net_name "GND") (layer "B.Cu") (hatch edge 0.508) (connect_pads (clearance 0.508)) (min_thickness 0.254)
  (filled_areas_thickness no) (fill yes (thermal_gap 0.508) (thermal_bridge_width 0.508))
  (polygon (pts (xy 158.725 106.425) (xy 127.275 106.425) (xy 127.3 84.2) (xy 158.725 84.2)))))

